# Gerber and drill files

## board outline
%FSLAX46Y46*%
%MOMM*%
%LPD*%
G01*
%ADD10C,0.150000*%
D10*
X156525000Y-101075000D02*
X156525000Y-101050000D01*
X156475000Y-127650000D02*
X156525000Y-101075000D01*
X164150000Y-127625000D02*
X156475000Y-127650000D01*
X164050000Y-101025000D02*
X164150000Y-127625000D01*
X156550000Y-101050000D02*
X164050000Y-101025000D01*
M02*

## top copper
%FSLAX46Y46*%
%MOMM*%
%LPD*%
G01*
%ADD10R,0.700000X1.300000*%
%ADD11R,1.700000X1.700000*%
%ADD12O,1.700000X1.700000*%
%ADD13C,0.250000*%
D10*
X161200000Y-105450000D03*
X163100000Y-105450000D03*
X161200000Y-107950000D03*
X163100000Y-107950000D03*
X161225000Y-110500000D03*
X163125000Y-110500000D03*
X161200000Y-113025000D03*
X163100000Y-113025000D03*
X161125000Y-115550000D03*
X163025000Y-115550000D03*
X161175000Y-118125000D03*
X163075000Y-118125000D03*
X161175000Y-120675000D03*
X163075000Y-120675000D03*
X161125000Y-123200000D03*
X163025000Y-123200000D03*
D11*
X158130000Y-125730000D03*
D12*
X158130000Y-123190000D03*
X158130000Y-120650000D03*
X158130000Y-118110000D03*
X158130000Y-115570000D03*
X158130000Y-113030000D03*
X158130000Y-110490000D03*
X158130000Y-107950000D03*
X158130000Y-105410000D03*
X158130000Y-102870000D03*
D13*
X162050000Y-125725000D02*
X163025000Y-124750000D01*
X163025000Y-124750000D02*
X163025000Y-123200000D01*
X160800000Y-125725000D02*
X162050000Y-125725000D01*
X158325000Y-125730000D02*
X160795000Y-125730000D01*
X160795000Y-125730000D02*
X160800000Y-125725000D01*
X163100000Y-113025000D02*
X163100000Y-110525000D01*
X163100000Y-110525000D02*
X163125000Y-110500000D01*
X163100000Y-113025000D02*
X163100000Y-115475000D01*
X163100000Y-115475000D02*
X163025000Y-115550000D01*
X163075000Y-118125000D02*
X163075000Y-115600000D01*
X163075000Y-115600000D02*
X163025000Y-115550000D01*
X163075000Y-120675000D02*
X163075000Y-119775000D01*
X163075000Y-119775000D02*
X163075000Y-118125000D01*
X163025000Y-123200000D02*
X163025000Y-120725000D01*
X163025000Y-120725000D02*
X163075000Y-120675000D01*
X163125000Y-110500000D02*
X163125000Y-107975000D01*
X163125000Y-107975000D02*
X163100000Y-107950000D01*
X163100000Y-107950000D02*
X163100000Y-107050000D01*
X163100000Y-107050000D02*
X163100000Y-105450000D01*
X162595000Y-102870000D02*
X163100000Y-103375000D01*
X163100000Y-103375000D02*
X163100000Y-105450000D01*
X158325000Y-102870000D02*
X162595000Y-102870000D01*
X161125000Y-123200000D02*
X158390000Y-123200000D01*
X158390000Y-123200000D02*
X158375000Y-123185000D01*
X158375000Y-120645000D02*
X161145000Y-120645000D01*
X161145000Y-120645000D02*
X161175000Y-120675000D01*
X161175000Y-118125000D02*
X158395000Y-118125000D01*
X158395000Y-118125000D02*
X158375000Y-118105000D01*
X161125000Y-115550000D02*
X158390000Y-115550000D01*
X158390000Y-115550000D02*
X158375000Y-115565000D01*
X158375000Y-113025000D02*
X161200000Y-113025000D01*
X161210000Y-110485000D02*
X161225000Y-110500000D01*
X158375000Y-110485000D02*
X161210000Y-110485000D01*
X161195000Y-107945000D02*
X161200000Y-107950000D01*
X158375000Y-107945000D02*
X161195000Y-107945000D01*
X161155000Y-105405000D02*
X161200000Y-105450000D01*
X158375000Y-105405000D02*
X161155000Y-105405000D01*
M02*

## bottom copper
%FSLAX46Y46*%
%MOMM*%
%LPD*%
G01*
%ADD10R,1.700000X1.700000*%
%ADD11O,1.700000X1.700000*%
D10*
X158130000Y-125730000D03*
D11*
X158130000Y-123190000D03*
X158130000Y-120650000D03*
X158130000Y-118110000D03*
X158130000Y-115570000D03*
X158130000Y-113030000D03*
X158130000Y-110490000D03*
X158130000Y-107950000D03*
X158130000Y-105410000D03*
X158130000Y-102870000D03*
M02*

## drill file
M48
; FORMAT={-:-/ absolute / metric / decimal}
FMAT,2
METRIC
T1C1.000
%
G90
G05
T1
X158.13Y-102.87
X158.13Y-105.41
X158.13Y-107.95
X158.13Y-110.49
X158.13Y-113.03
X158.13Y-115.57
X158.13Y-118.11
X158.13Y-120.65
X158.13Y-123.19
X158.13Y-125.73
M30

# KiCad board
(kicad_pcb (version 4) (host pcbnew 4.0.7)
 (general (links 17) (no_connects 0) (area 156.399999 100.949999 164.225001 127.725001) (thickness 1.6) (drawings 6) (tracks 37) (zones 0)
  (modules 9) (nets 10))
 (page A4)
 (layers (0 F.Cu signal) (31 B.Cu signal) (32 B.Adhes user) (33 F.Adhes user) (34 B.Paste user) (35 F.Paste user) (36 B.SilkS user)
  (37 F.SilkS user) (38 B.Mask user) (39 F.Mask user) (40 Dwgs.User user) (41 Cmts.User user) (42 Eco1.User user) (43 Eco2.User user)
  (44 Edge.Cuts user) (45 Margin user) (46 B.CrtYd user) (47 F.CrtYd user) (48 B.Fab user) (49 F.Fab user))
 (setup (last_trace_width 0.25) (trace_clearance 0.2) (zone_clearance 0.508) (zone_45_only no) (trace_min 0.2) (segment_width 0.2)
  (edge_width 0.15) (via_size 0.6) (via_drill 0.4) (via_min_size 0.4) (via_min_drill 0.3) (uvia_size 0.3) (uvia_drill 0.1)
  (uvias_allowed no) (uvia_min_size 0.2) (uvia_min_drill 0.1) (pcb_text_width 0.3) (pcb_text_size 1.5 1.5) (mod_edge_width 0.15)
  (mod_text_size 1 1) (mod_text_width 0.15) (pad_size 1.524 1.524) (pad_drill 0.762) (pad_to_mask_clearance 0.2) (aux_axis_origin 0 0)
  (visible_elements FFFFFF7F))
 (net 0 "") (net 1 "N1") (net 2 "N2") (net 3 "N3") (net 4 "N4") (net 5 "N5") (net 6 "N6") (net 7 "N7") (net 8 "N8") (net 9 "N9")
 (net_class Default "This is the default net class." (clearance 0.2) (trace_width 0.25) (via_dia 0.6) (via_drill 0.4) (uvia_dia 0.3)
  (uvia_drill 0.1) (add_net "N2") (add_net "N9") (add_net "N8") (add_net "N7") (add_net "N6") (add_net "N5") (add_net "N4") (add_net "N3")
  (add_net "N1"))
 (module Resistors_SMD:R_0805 (layer F.Cu) (at 162.15 105.45)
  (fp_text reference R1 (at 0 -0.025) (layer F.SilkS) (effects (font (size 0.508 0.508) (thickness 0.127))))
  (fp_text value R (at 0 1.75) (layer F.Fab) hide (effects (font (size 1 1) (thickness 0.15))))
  (pad 1 smd rect (at -0.95 0) (size 0.7 1.3) (layers F.Cu F.Paste F.Mask) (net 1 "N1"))
  (pad 2 smd rect (at 0.95 0) (size 0.7 1.3) (layers F.Cu F.Paste F.Mask) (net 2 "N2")))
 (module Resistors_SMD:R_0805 (layer F.Cu) (at 162.15 107.95)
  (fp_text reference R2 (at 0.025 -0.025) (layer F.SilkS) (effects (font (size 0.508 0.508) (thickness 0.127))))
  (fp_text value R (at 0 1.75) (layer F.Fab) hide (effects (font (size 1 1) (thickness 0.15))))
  (pad 1 smd rect (at -0.95 0) (size 0.7 1.3) (layers F.Cu F.Paste F.Mask) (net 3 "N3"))
  (pad 2 smd rect (at 0.95 0) (size 0.7 1.3) (layers F.Cu F.Paste F.Mask) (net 2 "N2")))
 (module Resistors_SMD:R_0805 (layer F.Cu) (at 162.175 110.5)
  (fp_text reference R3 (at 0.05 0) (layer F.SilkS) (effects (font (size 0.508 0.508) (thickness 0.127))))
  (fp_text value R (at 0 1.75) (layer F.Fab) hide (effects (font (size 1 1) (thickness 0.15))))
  (pad 1 smd rect (at -0.95 0) (size 0.7 1.3) (layers F.Cu F.Paste F.Mask) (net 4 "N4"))
  (pad 2 smd rect (at 0.95 0) (size 0.7 1.3) (layers F.Cu F.Paste F.Mask) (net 2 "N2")))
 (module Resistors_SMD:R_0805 (layer F.Cu) (at 162.15 113.025)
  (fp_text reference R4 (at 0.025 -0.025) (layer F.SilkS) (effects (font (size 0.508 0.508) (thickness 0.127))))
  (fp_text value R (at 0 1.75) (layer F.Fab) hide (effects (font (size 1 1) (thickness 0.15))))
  (pad 1 smd rect (at -0.95 0) (size 0.7 1.3) (layers F.Cu F.Paste F.Mask) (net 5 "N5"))
  (pad 2 smd rect (at 0.95 0) (size 0.7 1.3) (layers F.Cu F.Paste F.Mask) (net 2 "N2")))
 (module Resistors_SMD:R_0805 (layer F.Cu) (at 162.075 115.55)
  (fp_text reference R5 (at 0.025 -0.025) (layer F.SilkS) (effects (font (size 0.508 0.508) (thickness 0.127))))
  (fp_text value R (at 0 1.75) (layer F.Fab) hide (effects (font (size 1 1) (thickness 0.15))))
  (pad 1 smd rect (at -0.95 0) (size 0.7 1.3) (layers F.Cu F.Paste F.Mask) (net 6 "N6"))
  (pad 2 smd rect (at 0.95 0) (size 0.7 1.3) (layers F.Cu F.Paste F.Mask) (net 2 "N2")))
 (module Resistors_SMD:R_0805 (layer F.Cu) (at 162.125 118.125)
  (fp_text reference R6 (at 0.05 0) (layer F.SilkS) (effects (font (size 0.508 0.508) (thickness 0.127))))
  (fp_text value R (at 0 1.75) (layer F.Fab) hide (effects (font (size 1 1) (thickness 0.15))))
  (pad 1 smd rect (at -0.95 0) (size 0.7 1.3) (layers F.Cu F.Paste F.Mask) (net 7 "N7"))
  (pad 2 smd rect (at 0.95 0) (size 0.7 1.3) (layers F.Cu F.Paste F.Mask) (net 2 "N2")))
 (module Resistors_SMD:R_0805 (layer F.Cu) (at 162.125 120.675)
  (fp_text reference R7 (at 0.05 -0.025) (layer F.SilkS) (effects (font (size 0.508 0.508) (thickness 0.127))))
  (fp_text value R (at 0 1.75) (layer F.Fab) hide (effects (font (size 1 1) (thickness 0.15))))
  (pad 1 smd rect (at -0.95 0) (size 0.7 1.3) (layers F.Cu F.Paste F.Mask) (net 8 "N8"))
  (pad 2 smd rect (at 0.95 0) (size 0.7 1.3) (layers F.Cu F.Paste F.Mask) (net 2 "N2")))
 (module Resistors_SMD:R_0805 (layer F.Cu) (at 162.075 123.2)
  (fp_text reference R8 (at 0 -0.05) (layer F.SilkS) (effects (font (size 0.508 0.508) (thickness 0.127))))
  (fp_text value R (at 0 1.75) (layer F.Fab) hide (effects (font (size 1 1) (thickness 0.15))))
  (pad 1 smd rect (at -0.95 0) (size 0.7 1.3) (layers F.Cu F.Paste F.Mask) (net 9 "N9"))
  (pad 2 smd rect (at 0.95 0) (size 0.7 1.3) (layers F.Cu F.Paste F.Mask) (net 2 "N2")))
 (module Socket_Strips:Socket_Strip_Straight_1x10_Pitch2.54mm (layer B.Cu) (at 158.13 125.73)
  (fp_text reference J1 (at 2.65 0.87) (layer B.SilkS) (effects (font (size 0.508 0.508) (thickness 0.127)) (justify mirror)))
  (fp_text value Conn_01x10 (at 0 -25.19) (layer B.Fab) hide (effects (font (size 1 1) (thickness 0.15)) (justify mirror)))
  (pad 1 thru_hole rect (at 0 0) (size 1.7 1.7) (drill 1) (layers *.Cu *.Mask) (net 2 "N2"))
  (pad 2 thru_hole oval (at 0 -2.54) (size 1.7 1.7) (drill 1) (layers *.Cu *.Mask) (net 9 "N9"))
  (pad 3 thru_hole oval (at 0 -5.08) (size 1.7 1.7) (drill 1) (layers *.Cu *.Mask) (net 8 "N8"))
  (pad 4 thru_hole oval (at 0 -7.62) (size 1.7 1.7) (drill 1) (layers *.Cu *.Mask) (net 7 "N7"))
  (pad 5 thru_hole oval (at 0 -10.16) (size 1.7 1.7) (drill 1) (layers *.Cu *.Mask) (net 6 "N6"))
  (pad 6 thru_hole oval (at 0 -12.7) (size 1.7 1.7) (drill 1) (layers *.Cu *.Mask) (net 5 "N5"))
  (pad 7 thru_hole oval (at 0 -15.24) (size 1.7 1.7) (drill 1) (layers *.Cu *.Mask) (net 4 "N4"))
  (pad 8 thru_hole oval (at 0 -17.78) (size 1.7 1.7) (drill 1) (layers *.Cu *.Mask) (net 3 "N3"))
  (pad 9 thru_hole oval (at 0 -20.32) (size 1.7 1.7) (drill 1) (layers *.Cu *.Mask) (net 1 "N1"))
  (pad 10 thru_hole oval (at 0 -22.86) (size 1.7 1.7) (drill 1) (layers *.Cu *.Mask) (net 2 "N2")))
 (gr_line (start 156.525 101.075) (end 156.525 101.05) (layer Edge.Cuts) (width 0.15))
 (gr_line (start 156.475 127.65) (end 156.525 101.075) (layer Edge.Cuts) (width 0.15))
 (gr_line (start 164.15 127.625) (end 156.475 127.65) (layer Edge.Cuts) (width 0.15))
 (gr_line (start 164.05 101.025) (end 164.15 127.625) (layer Edge.Cuts) (width 0.15))
 (gr_line (start 156.55 101.05) (end 164.05 101.025) (layer Edge.Cuts) (width 0.15))
 (segment (start 162.05 125.725) (end 163.025 124.75) (width 0.25) (layer F.Cu) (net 2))
 (segment (start 163.025 124.75) (end 163.025 123.2) (width 0.25) (layer F.Cu) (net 2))
 (segment (start 160.8 125.725) (end 162.05 125.725) (width 0.25) (layer F.Cu) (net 2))
 (segment (start 158.325 125.73) (end 160.795 125.73) (width 0.25) (layer F.Cu) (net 2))
 (segment (start 160.795 125.73) (end 160.8 125.725) (width 0.25) (layer F.Cu) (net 2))
 (segment (start 163.1 113.025) (end 163.1 110.525) (width 0.25) (layer F.Cu) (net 2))
 (segment (start 163.1 110.525) (end 163.125 110.5) (width 0.25) (layer F.Cu) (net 2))
 (segment (start 163.1 113.025) (end 163.1 115.475) (width 0.25) (layer F.Cu) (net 2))
 (segment (start 163.1 115.475) (end 163.025 115.55) (width 0.25) (layer F.Cu) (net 2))
 (segment (start 163.075 118.125) (end 163.075 115.6) (width 0.25) (layer F.Cu) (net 2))
 (segment (start 163.075 115.6) (end 163.025 115.55) (width 0.25) (layer F.Cu) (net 2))
 (segment (start 163.075 120.675) (end 163.075 119.775) (width 0.25) (layer F.Cu) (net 2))
 (segment (start 163.075 119.775) (end 163.075 118.125) (width 0.25) (layer F.Cu) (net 2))
 (segment (start 163.025 123.2) (end 163.025 120.725) (width 0.25) (layer F.Cu) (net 2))
 (segment (start 163.025 120.725) (end 163.075 120.675) (width 0.25) (layer F.Cu) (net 2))
 (segment (start 163.125 110.5) (end 163.125 107.975) (width 0.25) (layer F.Cu) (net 2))
 (segment (start 163.125 107.975) (end 163.1 107.95) (width 0.25) (layer F.Cu) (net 2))
 (segment (start 163.1 107.95) (end 163.1 107.05) (width 0.25) (layer F.Cu) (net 2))
 (segment (start 163.1 107.05) (end 163.1 105.45) (width 0.25) (layer F.Cu) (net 2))
 (segment (start 162.595 102.87) (end 163.1 103.375) (width 0.25) (layer F.Cu) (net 2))
 (segment (start 163.1 103.375) (end 163.1 105.45) (width 0.25) (layer F.Cu) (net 2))
 (segment (start 158.325 102.87) (end 162.595 102.87) (width 0.25) (layer F.Cu) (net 2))
 (segment (start 161.125 123.2) (end 158.39 123.2) (width 0.25) (layer F.Cu) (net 9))
 (segment (start 158.39 123.2) (end 158.375 123.185) (width 0.25) (layer F.Cu) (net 9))
 (segment (start 158.375 120.645) (end 161.145 120.645) (width 0.25) (layer F.Cu) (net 8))
 (segment (start 161.145 120.645) (end 161.175 120.675) (width 0.25) (layer F.Cu) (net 8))
 (segment (start 161.175 118.125) (end 158.395 118.125) (width 0.25) (layer F.Cu) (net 7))
 (segment (start 158.395 118.125) (end 158.375 118.105) (width 0.25) (layer F.Cu) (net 7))
 (segment (start 161.125 115.55) (end 158.39 115.55) (width 0.25) (layer F.Cu) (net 6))
 (segment (start 158.39 115.55) (end 158.375 115.565) (width 0.25) (layer F.Cu) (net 6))
 (segment (start 158.375 113.025) (end 161.2 113.025) (width 0.25) (layer F.Cu) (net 5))
 (segment (start 161.21 110.485) (end 161.225 110.5) (width 0.25) (layer F.Cu) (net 4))
 (segment (start 158.375 110.485) (end 161.21 110.485) (width 0.25) (layer F.Cu) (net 4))
 (segment (start 161.195 107.945) (end 161.2 107.95) (width 0.25) (layer F.Cu) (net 3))
 (segment (start 158.375 107.945) (end 161.195 107.945) (width 0.25) (layer F.Cu) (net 3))
 (segment (start 161.155 105.405) (end 161.2 105.45) (width 0.25) (layer F.Cu) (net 1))
 (segment (start 158.375 105.405) (end 161.155 105.405) (width 0.25) (layer F.Cu) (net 1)))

